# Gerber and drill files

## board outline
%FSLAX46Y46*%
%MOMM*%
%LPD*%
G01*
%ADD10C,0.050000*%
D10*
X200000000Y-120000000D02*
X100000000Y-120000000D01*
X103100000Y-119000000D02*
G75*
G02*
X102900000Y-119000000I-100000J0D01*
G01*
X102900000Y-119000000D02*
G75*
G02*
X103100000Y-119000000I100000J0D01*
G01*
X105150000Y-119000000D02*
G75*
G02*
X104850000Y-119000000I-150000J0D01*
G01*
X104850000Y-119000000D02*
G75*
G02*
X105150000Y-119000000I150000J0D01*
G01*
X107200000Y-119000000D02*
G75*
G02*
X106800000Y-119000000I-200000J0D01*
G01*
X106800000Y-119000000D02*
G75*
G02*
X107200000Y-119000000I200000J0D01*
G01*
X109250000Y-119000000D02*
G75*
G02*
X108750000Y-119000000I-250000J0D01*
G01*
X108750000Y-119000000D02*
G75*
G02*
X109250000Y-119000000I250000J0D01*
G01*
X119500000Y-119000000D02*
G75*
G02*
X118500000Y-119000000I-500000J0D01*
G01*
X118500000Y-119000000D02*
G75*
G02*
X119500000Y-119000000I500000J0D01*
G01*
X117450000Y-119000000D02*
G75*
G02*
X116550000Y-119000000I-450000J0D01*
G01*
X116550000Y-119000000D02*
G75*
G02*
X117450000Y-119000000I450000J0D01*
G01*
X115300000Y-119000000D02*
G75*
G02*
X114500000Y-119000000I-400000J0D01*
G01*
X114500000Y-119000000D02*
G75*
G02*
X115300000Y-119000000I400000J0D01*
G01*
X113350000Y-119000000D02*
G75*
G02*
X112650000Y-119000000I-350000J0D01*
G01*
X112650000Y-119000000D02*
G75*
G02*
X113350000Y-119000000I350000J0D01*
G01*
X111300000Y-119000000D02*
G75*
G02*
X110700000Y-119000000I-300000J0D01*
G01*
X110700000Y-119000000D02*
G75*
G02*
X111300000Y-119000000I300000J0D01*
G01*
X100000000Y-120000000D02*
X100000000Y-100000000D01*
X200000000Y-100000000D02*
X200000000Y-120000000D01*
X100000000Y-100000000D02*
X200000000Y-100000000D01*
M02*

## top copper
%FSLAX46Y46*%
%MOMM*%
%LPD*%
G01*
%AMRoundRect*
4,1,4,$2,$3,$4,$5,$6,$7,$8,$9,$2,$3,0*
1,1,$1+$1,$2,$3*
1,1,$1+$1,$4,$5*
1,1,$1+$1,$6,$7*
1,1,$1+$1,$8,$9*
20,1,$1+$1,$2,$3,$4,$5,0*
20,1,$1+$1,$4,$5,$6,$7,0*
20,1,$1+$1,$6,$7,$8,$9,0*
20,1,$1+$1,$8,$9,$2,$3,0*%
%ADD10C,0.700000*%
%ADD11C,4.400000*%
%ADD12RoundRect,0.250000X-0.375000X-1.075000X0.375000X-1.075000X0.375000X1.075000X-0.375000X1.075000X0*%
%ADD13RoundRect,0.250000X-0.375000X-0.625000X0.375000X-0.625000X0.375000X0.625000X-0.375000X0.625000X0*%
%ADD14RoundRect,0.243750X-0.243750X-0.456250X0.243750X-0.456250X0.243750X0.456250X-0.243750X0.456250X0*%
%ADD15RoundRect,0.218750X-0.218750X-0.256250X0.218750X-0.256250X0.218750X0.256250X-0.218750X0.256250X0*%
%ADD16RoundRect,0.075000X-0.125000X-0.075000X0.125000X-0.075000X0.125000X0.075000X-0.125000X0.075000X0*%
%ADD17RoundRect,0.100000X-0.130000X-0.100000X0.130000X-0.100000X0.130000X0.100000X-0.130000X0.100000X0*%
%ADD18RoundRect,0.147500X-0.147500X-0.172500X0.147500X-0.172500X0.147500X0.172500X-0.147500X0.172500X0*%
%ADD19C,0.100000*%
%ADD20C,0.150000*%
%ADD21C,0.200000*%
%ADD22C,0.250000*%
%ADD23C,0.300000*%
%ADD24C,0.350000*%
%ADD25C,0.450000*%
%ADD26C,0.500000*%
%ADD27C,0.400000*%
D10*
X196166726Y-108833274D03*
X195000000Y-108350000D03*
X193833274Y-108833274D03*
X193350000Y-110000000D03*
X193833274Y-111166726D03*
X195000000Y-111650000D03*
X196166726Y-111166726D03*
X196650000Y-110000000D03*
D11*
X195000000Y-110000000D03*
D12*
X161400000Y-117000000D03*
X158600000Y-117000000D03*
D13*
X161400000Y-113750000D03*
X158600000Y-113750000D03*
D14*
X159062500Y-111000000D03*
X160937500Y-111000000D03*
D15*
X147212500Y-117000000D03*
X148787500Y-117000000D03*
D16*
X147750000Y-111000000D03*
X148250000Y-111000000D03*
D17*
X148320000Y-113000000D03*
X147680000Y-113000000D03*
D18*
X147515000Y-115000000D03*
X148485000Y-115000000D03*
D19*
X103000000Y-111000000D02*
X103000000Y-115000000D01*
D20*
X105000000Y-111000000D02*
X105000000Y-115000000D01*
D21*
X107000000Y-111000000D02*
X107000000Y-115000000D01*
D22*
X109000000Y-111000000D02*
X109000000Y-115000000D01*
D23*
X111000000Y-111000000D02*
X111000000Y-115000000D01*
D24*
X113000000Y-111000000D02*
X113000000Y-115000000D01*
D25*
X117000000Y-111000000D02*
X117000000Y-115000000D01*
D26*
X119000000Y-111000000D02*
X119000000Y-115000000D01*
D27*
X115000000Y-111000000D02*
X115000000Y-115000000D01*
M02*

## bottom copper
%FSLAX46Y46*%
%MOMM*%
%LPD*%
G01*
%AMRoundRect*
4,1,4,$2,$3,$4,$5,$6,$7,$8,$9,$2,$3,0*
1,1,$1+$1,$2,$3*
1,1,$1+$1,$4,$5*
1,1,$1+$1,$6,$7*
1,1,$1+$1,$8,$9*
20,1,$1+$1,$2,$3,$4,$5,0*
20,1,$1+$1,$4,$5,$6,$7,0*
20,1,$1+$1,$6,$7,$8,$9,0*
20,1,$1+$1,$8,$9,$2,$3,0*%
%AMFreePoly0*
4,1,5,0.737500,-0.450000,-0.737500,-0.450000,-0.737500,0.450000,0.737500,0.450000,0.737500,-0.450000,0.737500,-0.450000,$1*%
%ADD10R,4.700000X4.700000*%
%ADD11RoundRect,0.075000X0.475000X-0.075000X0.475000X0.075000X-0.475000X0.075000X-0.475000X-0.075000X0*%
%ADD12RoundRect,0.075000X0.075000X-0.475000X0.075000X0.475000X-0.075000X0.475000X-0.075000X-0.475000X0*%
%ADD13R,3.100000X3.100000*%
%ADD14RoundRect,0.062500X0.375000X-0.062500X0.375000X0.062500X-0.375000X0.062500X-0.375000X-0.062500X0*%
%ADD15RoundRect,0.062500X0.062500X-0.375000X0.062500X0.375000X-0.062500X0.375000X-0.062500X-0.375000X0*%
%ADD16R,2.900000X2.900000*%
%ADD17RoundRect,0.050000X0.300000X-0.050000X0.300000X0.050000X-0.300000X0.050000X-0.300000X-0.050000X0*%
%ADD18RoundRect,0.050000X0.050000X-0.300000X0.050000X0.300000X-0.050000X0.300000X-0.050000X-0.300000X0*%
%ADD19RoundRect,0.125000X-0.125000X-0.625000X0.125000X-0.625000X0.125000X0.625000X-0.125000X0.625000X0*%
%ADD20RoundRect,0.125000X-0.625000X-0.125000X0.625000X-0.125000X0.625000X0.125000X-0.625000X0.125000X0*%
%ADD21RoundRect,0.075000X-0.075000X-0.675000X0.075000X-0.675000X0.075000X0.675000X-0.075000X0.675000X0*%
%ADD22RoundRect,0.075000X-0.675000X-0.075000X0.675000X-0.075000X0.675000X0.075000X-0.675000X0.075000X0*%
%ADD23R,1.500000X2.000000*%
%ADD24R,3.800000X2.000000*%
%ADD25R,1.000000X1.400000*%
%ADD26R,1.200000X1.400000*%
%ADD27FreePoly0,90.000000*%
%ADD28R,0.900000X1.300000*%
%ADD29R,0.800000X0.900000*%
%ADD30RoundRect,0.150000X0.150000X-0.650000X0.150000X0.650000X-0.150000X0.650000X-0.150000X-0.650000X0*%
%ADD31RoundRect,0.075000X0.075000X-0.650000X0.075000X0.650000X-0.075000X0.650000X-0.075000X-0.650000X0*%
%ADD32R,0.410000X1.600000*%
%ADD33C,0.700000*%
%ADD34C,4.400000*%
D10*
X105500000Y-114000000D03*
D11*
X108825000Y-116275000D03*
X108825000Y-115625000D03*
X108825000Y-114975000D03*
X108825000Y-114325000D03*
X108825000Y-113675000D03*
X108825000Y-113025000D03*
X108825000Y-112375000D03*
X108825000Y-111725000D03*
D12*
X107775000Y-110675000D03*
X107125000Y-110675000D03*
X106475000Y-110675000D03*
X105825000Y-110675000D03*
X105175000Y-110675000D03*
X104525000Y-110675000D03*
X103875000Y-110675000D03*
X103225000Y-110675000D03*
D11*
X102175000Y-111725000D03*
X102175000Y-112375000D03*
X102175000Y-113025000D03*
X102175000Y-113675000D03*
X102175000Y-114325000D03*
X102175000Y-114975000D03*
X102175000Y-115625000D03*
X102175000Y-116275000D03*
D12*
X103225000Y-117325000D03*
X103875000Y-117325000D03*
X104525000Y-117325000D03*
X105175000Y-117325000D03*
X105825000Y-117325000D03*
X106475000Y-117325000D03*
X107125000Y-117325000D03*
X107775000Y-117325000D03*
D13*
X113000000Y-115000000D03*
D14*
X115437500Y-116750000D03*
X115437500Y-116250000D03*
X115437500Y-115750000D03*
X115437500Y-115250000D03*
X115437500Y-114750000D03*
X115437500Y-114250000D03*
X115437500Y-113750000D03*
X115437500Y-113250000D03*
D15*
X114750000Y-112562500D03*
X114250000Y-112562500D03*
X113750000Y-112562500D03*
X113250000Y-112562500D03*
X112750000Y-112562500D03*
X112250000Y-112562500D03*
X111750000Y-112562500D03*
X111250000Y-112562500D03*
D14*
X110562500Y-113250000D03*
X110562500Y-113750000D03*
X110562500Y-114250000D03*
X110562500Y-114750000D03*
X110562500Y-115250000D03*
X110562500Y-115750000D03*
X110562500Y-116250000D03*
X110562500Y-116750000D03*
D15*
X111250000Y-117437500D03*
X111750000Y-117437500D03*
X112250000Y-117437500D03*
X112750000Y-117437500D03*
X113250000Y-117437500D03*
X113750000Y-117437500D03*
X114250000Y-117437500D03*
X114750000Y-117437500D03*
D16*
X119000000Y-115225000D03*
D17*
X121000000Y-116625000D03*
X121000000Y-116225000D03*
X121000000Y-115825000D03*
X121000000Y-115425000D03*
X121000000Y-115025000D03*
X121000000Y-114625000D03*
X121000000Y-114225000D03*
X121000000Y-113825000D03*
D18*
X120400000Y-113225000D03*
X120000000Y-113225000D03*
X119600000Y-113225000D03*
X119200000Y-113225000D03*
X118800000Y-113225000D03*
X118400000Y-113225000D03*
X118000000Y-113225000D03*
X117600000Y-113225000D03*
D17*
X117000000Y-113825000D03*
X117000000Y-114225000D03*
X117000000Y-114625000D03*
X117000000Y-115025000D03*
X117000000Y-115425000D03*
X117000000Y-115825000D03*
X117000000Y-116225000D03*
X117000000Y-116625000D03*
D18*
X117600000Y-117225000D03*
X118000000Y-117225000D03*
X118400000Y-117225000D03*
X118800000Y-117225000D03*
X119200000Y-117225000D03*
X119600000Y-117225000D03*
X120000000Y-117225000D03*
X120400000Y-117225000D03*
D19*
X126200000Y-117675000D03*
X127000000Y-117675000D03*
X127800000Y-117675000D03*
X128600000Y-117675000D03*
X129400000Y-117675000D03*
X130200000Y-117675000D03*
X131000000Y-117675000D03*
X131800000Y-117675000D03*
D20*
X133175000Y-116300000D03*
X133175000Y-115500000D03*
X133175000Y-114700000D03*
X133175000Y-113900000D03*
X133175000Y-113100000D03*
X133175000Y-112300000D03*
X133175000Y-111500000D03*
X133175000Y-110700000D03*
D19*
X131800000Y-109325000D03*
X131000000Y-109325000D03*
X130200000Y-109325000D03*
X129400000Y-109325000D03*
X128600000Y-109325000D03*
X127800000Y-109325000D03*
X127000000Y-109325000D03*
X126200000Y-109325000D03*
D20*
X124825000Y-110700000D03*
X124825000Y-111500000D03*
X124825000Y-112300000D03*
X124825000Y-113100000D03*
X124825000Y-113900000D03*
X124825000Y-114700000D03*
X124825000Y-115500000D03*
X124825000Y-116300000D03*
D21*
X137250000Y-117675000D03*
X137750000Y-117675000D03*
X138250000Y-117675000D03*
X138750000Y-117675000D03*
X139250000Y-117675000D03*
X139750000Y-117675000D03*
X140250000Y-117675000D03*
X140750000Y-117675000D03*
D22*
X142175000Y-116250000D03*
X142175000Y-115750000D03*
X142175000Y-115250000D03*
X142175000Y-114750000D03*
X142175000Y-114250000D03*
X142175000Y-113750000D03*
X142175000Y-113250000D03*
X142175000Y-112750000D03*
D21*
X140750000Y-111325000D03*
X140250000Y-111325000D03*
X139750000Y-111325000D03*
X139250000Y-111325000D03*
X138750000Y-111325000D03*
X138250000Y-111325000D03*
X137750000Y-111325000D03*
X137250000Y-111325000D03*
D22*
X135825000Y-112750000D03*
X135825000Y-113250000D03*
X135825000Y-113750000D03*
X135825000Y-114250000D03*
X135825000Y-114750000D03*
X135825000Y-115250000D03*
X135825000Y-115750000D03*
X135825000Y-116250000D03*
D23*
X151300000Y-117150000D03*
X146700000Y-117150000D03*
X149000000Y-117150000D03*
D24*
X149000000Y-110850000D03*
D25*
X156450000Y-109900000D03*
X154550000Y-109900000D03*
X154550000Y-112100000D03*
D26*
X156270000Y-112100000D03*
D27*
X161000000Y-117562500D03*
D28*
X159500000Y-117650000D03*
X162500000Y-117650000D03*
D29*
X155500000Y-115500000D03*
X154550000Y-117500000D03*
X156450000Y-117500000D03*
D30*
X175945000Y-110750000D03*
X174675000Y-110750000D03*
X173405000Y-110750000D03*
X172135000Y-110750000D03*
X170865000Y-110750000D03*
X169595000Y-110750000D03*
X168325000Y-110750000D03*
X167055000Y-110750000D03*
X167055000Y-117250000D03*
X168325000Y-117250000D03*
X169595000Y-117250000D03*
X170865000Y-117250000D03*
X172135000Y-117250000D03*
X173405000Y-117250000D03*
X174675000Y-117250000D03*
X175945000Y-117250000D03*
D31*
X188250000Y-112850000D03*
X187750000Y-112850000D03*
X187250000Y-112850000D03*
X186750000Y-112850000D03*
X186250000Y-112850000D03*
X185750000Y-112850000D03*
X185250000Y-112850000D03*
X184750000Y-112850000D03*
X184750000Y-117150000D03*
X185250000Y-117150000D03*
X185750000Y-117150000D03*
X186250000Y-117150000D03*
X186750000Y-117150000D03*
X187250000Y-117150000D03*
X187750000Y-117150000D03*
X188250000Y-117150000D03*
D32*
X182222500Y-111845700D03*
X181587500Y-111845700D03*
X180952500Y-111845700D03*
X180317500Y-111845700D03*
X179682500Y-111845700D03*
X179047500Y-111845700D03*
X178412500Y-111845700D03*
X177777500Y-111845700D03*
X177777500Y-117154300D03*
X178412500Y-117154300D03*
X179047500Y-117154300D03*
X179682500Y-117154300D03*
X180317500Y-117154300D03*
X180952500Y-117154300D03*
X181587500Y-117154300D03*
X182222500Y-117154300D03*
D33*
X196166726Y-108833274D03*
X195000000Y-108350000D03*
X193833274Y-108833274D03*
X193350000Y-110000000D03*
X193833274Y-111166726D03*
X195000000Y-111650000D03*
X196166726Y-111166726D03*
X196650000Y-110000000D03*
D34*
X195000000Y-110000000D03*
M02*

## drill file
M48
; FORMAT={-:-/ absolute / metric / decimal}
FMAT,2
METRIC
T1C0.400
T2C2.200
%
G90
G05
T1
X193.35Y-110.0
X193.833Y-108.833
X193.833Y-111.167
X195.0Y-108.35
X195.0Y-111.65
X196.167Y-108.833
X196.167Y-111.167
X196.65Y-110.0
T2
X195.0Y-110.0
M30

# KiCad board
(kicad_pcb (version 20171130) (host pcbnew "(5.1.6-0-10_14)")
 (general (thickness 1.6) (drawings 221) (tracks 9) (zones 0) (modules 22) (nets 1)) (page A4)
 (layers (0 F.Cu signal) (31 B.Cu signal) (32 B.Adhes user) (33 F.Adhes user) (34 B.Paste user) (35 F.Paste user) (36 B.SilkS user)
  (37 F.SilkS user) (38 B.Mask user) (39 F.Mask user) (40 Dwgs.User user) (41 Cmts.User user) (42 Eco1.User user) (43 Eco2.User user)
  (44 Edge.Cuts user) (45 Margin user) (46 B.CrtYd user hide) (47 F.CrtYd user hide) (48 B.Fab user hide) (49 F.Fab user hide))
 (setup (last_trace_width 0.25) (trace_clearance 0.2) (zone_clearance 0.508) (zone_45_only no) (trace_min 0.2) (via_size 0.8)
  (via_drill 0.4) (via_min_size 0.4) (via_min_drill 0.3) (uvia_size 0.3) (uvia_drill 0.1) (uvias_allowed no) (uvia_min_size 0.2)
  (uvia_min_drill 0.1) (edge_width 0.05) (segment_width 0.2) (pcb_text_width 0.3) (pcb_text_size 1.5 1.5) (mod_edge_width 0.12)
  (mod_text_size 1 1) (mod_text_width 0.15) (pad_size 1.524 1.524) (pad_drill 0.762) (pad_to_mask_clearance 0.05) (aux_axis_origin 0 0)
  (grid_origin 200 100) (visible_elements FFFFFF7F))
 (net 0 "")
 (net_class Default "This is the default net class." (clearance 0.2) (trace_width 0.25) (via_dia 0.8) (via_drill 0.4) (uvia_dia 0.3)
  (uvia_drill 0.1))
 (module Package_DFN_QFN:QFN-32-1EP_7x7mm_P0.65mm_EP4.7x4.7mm (layer B.Cu) (at 105.5 114 90)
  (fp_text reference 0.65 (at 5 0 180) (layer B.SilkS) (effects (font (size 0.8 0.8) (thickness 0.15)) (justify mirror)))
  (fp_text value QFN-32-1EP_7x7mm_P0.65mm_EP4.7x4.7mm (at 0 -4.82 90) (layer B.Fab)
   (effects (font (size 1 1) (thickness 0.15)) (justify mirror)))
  (pad "" smd roundrect (at 1.77 -1.77 90) (size 0.95 0.95) (layers B.Paste) (roundrect_rratio 0.25))
  (pad "" smd roundrect (at 1.77 -0.59 90) (size 0.95 0.95) (layers B.Paste) (roundrect_rratio 0.25))
  (pad "" smd roundrect (at 1.77 0.59 90) (size 0.95 0.95) (layers B.Paste) (roundrect_rratio 0.25))
  (pad "" smd roundrect (at 1.77 1.77 90) (size 0.95 0.95) (layers B.Paste) (roundrect_rratio 0.25))
  (pad "" smd roundrect (at 0.59 -1.77 90) (size 0.95 0.95) (layers B.Paste) (roundrect_rratio 0.25))
  (pad "" smd roundrect (at 0.59 -0.59 90) (size 0.95 0.95) (layers B.Paste) (roundrect_rratio 0.25))
  (pad "" smd roundrect (at 0.59 0.59 90) (size 0.95 0.95) (layers B.Paste) (roundrect_rratio 0.25))
  (pad "" smd roundrect (at 0.59 1.77 90) (size 0.95 0.95) (layers B.Paste) (roundrect_rratio 0.25))
  (pad "" smd roundrect (at -0.59 -1.77 90) (size 0.95 0.95) (layers B.Paste) (roundrect_rratio 0.25))
  (pad "" smd roundrect (at -0.59 -0.59 90) (size 0.95 0.95) (layers B.Paste) (roundrect_rratio 0.25))
  (pad "" smd roundrect (at -0.59 0.59 90) (size 0.95 0.95) (layers B.Paste) (roundrect_rratio 0.25))
  (pad "" smd roundrect (at -0.59 1.77 90) (size 0.95 0.95) (layers B.Paste) (roundrect_rratio 0.25))
  (pad "" smd roundrect (at -1.77 -1.77 90) (size 0.95 0.95) (layers B.Paste) (roundrect_rratio 0.25))
  (pad "" smd roundrect (at -1.77 -0.59 90) (size 0.95 0.95) (layers B.Paste) (roundrect_rratio 0.25))
  (pad "" smd roundrect (at -1.77 0.59 90) (size 0.95 0.95) (layers B.Paste) (roundrect_rratio 0.25))
  (pad "" smd roundrect (at -1.77 1.77 90) (size 0.95 0.95) (layers B.Paste) (roundrect_rratio 0.25))
  (pad 33 smd rect (at 0 0 90) (size 4.7 4.7) (layers B.Cu B.Mask))
  (pad 32 smd roundrect (at -2.275 3.325 90) (size 0.3 1.1) (layers B.Cu B.Paste B.Mask) (roundrect_rratio 0.25))
  (pad 31 smd roundrect (at -1.625 3.325 90) (size 0.3 1.1) (layers B.Cu B.Paste B.Mask) (roundrect_rratio 0.25))
  (pad 30 smd roundrect (at -0.975 3.325 90) (size 0.3 1.1) (layers B.Cu B.Paste B.Mask) (roundrect_rratio 0.25))
  (pad 29 smd roundrect (at -0.325 3.325 90) (size 0.3 1.1) (layers B.Cu B.Paste B.Mask) (roundrect_rratio 0.25))
  (pad 28 smd roundrect (at 0.325 3.325 90) (size 0.3 1.1) (layers B.Cu B.Paste B.Mask) (roundrect_rratio 0.25))
  (pad 27 smd roundrect (at 0.975 3.325 90) (size 0.3 1.1) (layers B.Cu B.Paste B.Mask) (roundrect_rratio 0.25))
  (pad 26 smd roundrect (at 1.625 3.325 90) (size 0.3 1.1) (layers B.Cu B.Paste B.Mask) (roundrect_rratio 0.25))
  (pad 25 smd roundrect (at 2.275 3.325 90) (size 0.3 1.1) (layers B.Cu B.Paste B.Mask) (roundrect_rratio 0.25))
  (pad 24 smd roundrect (at 3.325 2.275 90) (size 1.1 0.3) (layers B.Cu B.Paste B.Mask) (roundrect_rratio 0.25))
  (pad 23 smd roundrect (at 3.325 1.625 90) (size 1.1 0.3) (layers B.Cu B.Paste B.Mask) (roundrect_rratio 0.25))
  (pad 22 smd roundrect (at 3.325 0.975 90) (size 1.1 0.3) (layers B.Cu B.Paste B.Mask) (roundrect_rratio 0.25))
  (pad 21 smd roundrect (at 3.325 0.325 90) (size 1.1 0.3) (layers B.Cu B.Paste B.Mask) (roundrect_rratio 0.25))
  (pad 20 smd roundrect (at 3.325 -0.325 90) (size 1.1 0.3) (layers B.Cu B.Paste B.Mask) (roundrect_rratio 0.25))
  (pad 19 smd roundrect (at 3.325 -0.975 90) (size 1.1 0.3) (layers B.Cu B.Paste B.Mask) (roundrect_rratio 0.25))
  (pad 18 smd roundrect (at 3.325 -1.625 90) (size 1.1 0.3) (layers B.Cu B.Paste B.Mask) (roundrect_rratio 0.25))
  (pad 17 smd roundrect (at 3.325 -2.275 90) (size 1.1 0.3) (layers B.Cu B.Paste B.Mask) (roundrect_rratio 0.25))
  (pad 16 smd roundrect (at 2.275 -3.325 90) (size 0.3 1.1) (layers B.Cu B.Paste B.Mask) (roundrect_rratio 0.25))
  (pad 15 smd roundrect (at 1.625 -3.325 90) (size 0.3 1.1) (layers B.Cu B.Paste B.Mask) (roundrect_rratio 0.25))
  (pad 14 smd roundrect (at 0.975 -3.325 90) (size 0.3 1.1) (layers B.Cu B.Paste B.Mask) (roundrect_rratio 0.25))
  (pad 13 smd roundrect (at 0.325 -3.325 90) (size 0.3 1.1) (layers B.Cu B.Paste B.Mask) (roundrect_rratio 0.25))
  (pad 12 smd roundrect (at -0.325 -3.325 90) (size 0.3 1.1) (layers B.Cu B.Paste B.Mask) (roundrect_rratio 0.25))
  (pad 11 smd roundrect (at -0.975 -3.325 90) (size 0.3 1.1) (layers B.Cu B.Paste B.Mask) (roundrect_rratio 0.25))
  (pad 10 smd roundrect (at -1.625 -3.325 90) (size 0.3 1.1) (layers B.Cu B.Paste B.Mask) (roundrect_rratio 0.25))
  (pad 9 smd roundrect (at -2.275 -3.325 90) (size 0.3 1.1) (layers B.Cu B.Paste B.Mask) (roundrect_rratio 0.25))
  (pad 8 smd roundrect (at -3.325 -2.275 90) (size 1.1 0.3) (layers B.Cu B.Paste B.Mask) (roundrect_rratio 0.25))
  (pad 7 smd roundrect (at -3.325 -1.625 90) (size 1.1 0.3) (layers B.Cu B.Paste B.Mask) (roundrect_rratio 0.25))
  (pad 6 smd roundrect (at -3.325 -0.975 90) (size 1.1 0.3) (layers B.Cu B.Paste B.Mask) (roundrect_rratio 0.25))
  (pad 5 smd roundrect (at -3.325 -0.325 90) (size 1.1 0.3) (layers B.Cu B.Paste B.Mask) (roundrect_rratio 0.25))
  (pad 4 smd roundrect (at -3.325 0.325 90) (size 1.1 0.3) (layers B.Cu B.Paste B.Mask) (roundrect_rratio 0.25))
  (pad 3 smd roundrect (at -3.325 0.975 90) (size 1.1 0.3) (layers B.Cu B.Paste B.Mask) (roundrect_rratio 0.25))
  (pad 2 smd roundrect (at -3.325 1.625 90) (size 1.1 0.3) (layers B.Cu B.Paste B.Mask) (roundrect_rratio 0.25))
  (pad 1 smd roundrect (at -3.325 2.275 90) (size 1.1 0.3) (layers B.Cu B.Paste B.Mask) (roundrect_rratio 0.25)))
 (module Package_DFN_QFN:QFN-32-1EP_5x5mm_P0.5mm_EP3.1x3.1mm (layer B.Cu) (at 113 115 90)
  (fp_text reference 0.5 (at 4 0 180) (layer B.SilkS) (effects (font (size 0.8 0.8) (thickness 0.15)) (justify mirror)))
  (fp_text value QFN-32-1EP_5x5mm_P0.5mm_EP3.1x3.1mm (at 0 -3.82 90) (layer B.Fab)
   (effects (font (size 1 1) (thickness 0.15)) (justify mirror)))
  (pad "" smd roundrect (at 1.03 -1.03 90) (size 0.83 0.83) (layers B.Paste) (roundrect_rratio 0.25))
  (pad "" smd roundrect (at 1.03 0 90) (size 0.83 0.83) (layers B.Paste) (roundrect_rratio 0.25))
  (pad "" smd roundrect (at 1.03 1.03 90) (size 0.83 0.83) (layers B.Paste) (roundrect_rratio 0.25))
  (pad "" smd roundrect (at 0 -1.03 90) (size 0.83 0.83) (layers B.Paste) (roundrect_rratio 0.25))
  (pad "" smd roundrect (at 0 0 90) (size 0.83 0.83) (layers B.Paste) (roundrect_rratio 0.25))
  (pad "" smd roundrect (at 0 1.03 90) (size 0.83 0.83) (layers B.Paste) (roundrect_rratio 0.25))
  (pad "" smd roundrect (at -1.03 -1.03 90) (size 0.83 0.83) (layers B.Paste) (roundrect_rratio 0.25))
  (pad "" smd roundrect (at -1.03 0 90) (size 0.83 0.83) (layers B.Paste) (roundrect_rratio 0.25))
  (pad "" smd roundrect (at -1.03 1.03 90) (size 0.83 0.83) (layers B.Paste) (roundrect_rratio 0.25))
  (pad 33 smd rect (at 0 0 90) (size 3.1 3.1) (layers B.Cu B.Mask))
  (pad 32 smd roundrect (at -1.75 2.4375 90) (size 0.25 0.875) (layers B.Cu B.Paste B.Mask) (roundrect_rratio 0.25))
  (pad 31 smd roundrect (at -1.25 2.4375 90) (size 0.25 0.875) (layers B.Cu B.Paste B.Mask) (roundrect_rratio 0.25))
  (pad 30 smd roundrect (at -0.75 2.4375 90) (size 0.25 0.875) (layers B.Cu B.Paste B.Mask) (roundrect_rratio 0.25))
  (pad 29 smd roundrect (at -0.25 2.4375 90) (size 0.25 0.875) (layers B.Cu B.Paste B.Mask) (roundrect_rratio 0.25))
  (pad 28 smd roundrect (at 0.25 2.4375 90) (size 0.25 0.875) (layers B.Cu B.Paste B.Mask) (roundrect_rratio 0.25))
  (pad 27 smd roundrect (at 0.75 2.4375 90) (size 0.25 0.875) (layers B.Cu B.Paste B.Mask) (roundrect_rratio 0.25))
  (pad 26 smd roundrect (at 1.25 2.4375 90) (size 0.25 0.875) (layers B.Cu B.Paste B.Mask) (roundrect_rratio 0.25))
  (pad 25 smd roundrect (at 1.75 2.4375 90) (size 0.25 0.875) (layers B.Cu B.Paste B.Mask) (roundrect_rratio 0.25))
  (pad 24 smd roundrect (at 2.4375 1.75 90) (size 0.875 0.25) (layers B.Cu B.Paste B.Mask) (roundrect_rratio 0.25))
  (pad 23 smd roundrect (at 2.4375 1.25 90) (size 0.875 0.25) (layers B.Cu B.Paste B.Mask) (roundrect_rratio 0.25))
  (pad 22 smd roundrect (at 2.4375 0.75 90) (size 0.875 0.25) (layers B.Cu B.Paste B.Mask) (roundrect_rratio 0.25))
  (pad 21 smd roundrect (at 2.4375 0.25 90) (size 0.875 0.25) (layers B.Cu B.Paste B.Mask) (roundrect_rratio 0.25))
  (pad 20 smd roundrect (at 2.4375 -0.25 90) (size 0.875 0.25) (layers B.Cu B.Paste B.Mask) (roundrect_rratio 0.25))
  (pad 19 smd roundrect (at 2.4375 -0.75 90) (size 0.875 0.25) (layers B.Cu B.Paste B.Mask) (roundrect_rratio 0.25))
  (pad 18 smd roundrect (at 2.4375 -1.25 90) (size 0.875 0.25) (layers B.Cu B.Paste B.Mask) (roundrect_rratio 0.25))
  (pad 17 smd roundrect (at 2.4375 -1.75 90) (size 0.875 0.25) (layers B.Cu B.Paste B.Mask) (roundrect_rratio 0.25))
  (pad 16 smd roundrect (at 1.75 -2.4375 90) (size 0.25 0.875) (layers B.Cu B.Paste B.Mask) (roundrect_rratio 0.25))
  (pad 15 smd roundrect (at 1.25 -2.4375 90) (size 0.25 0.875) (layers B.Cu B.Paste B.Mask) (roundrect_rratio 0.25))
  (pad 14 smd roundrect (at 0.75 -2.4375 90) (size 0.25 0.875) (layers B.Cu B.Paste B.Mask) (roundrect_rratio 0.25))
  (pad 13 smd roundrect (at 0.25 -2.4375 90) (size 0.25 0.875) (layers B.Cu B.Paste B.Mask) (roundrect_rratio 0.25))
  (pad 12 smd roundrect (at -0.25 -2.4375 90) (size 0.25 0.875) (layers B.Cu B.Paste B.Mask) (roundrect_rratio 0.25))
  (pad 11 smd roundrect (at -0.75 -2.4375 90) (size 0.25 0.875) (layers B.Cu B.Paste B.Mask) (roundrect_rratio 0.25))
  (pad 10 smd roundrect (at -1.25 -2.4375 90) (size 0.25 0.875) (layers B.Cu B.Paste B.Mask) (roundrect_rratio 0.25))
  (pad 9 smd roundrect (at -1.75 -2.4375 90) (size 0.25 0.875) (layers B.Cu B.Paste B.Mask) (roundrect_rratio 0.25))
  (pad 8 smd roundrect (at -2.4375 -1.75 90) (size 0.875 0.25) (layers B.Cu B.Paste B.Mask) (roundrect_rratio 0.25))
  (pad 7 smd roundrect (at -2.4375 -1.25 90) (size 0.875 0.25) (layers B.Cu B.Paste B.Mask) (roundrect_rratio 0.25))
  (pad 6 smd roundrect (at -2.4375 -0.75 90) (size 0.875 0.25) (layers B.Cu B.Paste B.Mask) (roundrect_rratio 0.25))
  (pad 5 smd roundrect (at -2.4375 -0.25 90) (size 0.875 0.25) (layers B.Cu B.Paste B.Mask) (roundrect_rratio 0.25))
  (pad 4 smd roundrect (at -2.4375 0.25 90) (size 0.875 0.25) (layers B.Cu B.Paste B.Mask) (roundrect_rratio 0.25))
  (pad 3 smd roundrect (at -2.4375 0.75 90) (size 0.875 0.25) (layers B.Cu B.Paste B.Mask) (roundrect_rratio 0.25))
  (pad 2 smd roundrect (at -2.4375 1.25 90) (size 0.875 0.25) (layers B.Cu B.Paste B.Mask) (roundrect_rratio 0.25))
  (pad 1 smd roundrect (at -2.4375 1.75 90) (size 0.875 0.25) (layers B.Cu B.Paste B.Mask) (roundrect_rratio 0.25)))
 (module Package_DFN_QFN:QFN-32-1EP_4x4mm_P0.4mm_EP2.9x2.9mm (layer B.Cu) (at 119 115.225 90)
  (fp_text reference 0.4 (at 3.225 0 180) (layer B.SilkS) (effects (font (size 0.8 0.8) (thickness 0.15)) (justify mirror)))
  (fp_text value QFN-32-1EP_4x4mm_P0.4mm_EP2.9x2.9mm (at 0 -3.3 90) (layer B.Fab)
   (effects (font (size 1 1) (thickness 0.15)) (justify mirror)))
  (pad "" smd roundrect (at 0.725 -0.725 90) (size 1.17 1.17) (layers B.Paste) (roundrect_rratio 0.213675))
  (pad "" smd roundrect (at 0.725 0.725 90) (size 1.17 1.17) (layers B.Paste) (roundrect_rratio 0.213675))
  (pad "" smd roundrect (at -0.725 -0.725 90) (size 1.17 1.17) (layers B.Paste) (roundrect_rratio 0.213675))
  (pad "" smd roundrect (at -0.725 0.725 90) (size 1.17 1.17) (layers B.Paste) (roundrect_rratio 0.213675))
  (pad 33 smd rect (at 0 0 90) (size 2.9 2.9) (layers B.Cu B.Mask))
  (pad 32 smd roundrect (at -1.4 2 90) (size 0.2 0.7) (layers B.Cu B.Paste B.Mask) (roundrect_rratio 0.25))
  (pad 31 smd roundrect (at -1 2 90) (size 0.2 0.7) (layers B.Cu B.Paste B.Mask) (roundrect_rratio 0.25))
  (pad 30 smd roundrect (at -0.6 2 90) (size 0.2 0.7) (layers B.Cu B.Paste B.Mask) (roundrect_rratio 0.25))
  (pad 29 smd roundrect (at -0.2 2 90) (size 0.2 0.7) (layers B.Cu B.Paste B.Mask) (roundrect_rratio 0.25))
  (pad 28 smd roundrect (at 0.2 2 90) (size 0.2 0.7) (layers B.Cu B.Paste B.Mask) (roundrect_rratio 0.25))
  (pad 27 smd roundrect (at 0.6 2 90) (size 0.2 0.7) (layers B.Cu B.Paste B.Mask) (roundrect_rratio 0.25))
  (pad 26 smd roundrect (at 1 2 90) (size 0.2 0.7) (layers B.Cu B.Paste B.Mask) (roundrect_rratio 0.25))
  (pad 25 smd roundrect (at 1.4 2 90) (size 0.2 0.7) (layers B.Cu B.Paste B.Mask) (roundrect_rratio 0.25))
  (pad 24 smd roundrect (at 2 1.4 90) (size 0.7 0.2) (layers B.Cu B.Paste B.Mask) (roundrect_rratio 0.25))
  (pad 23 smd roundrect (at 2 1 90) (size 0.7 0.2) (layers B.Cu B.Paste B.Mask) (roundrect_rratio 0.25))
  (pad 22 smd roundrect (at 2 0.6 90) (size 0.7 0.2) (layers B.Cu B.Paste B.Mask) (roundrect_rratio 0.25))
  (pad 21 smd roundrect (at 2 0.2 90) (size 0.7 0.2) (layers B.Cu B.Paste B.Mask) (roundrect_rratio 0.25))
  (pad 20 smd roundrect (at 2 -0.2 90) (size 0.7 0.2) (layers B.Cu B.Paste B.Mask) (roundrect_rratio 0.25))
  (pad 19 smd roundrect (at 2 -0.6 90) (size 0.7 0.2) (layers B.Cu B.Paste B.Mask) (roundrect_rratio 0.25))
  (pad 18 smd roundrect (at 2 -1 90) (size 0.7 0.2) (layers B.Cu B.Paste B.Mask) (roundrect_rratio 0.25))
  (pad 17 smd roundrect (at 2 -1.4 90) (size 0.7 0.2) (layers B.Cu B.Paste B.Mask) (roundrect_rratio 0.25))
  (pad 16 smd roundrect (at 1.4 -2 90) (size 0.2 0.7) (layers B.Cu B.Paste B.Mask) (roundrect_rratio 0.25))
  (pad 15 smd roundrect (at 1 -2 90) (size 0.2 0.7) (layers B.Cu B.Paste B.Mask) (roundrect_rratio 0.25))
  (pad 14 smd roundrect (at 0.6 -2 90) (size 0.2 0.7) (layers B.Cu B.Paste B.Mask) (roundrect_rratio 0.25))
  (pad 13 smd roundrect (at 0.2 -2 90) (size 0.2 0.7) (layers B.Cu B.Paste B.Mask) (roundrect_rratio 0.25))
  (pad 12 smd roundrect (at -0.2 -2 90) (size 0.2 0.7) (layers B.Cu B.Paste B.Mask) (roundrect_rratio 0.25))
  (pad 11 smd roundrect (at -0.6 -2 90) (size 0.2 0.7) (layers B.Cu B.Paste B.Mask) (roundrect_rratio 0.25))
  (pad 10 smd roundrect (at -1 -2 90) (size 0.2 0.7) (layers B.Cu B.Paste B.Mask) (roundrect_rratio 0.25))
  (pad 9 smd roundrect (at -1.4 -2 90) (size 0.2 0.7) (layers B.Cu B.Paste B.Mask) (roundrect_rratio 0.25))
  (pad 8 smd roundrect (at -2 -1.4 90) (size 0.7 0.2) (layers B.Cu B.Paste B.Mask) (roundrect_rratio 0.25))
  (pad 7 smd roundrect (at -2 -1 90) (size 0.7 0.2) (layers B.Cu B.Paste B.Mask) (roundrect_rratio 0.25))
  (pad 6 smd roundrect (at -2 -0.6 90) (size 0.7 0.2) (layers B.Cu B.Paste B.Mask) (roundrect_rratio 0.25))
  (pad 5 smd roundrect (at -2 -0.2 90) (size 0.7 0.2) (layers B.Cu B.Paste B.Mask) (roundrect_rratio 0.25))
  (pad 4 smd roundrect (at -2 0.2 90) (size 0.7 0.2) (layers B.Cu B.Paste B.Mask) (roundrect_rratio 0.25))
  (pad 3 smd roundrect (at -2 0.6 90) (size 0.7 0.2) (layers B.Cu B.Paste B.Mask) (roundrect_rratio 0.25))
  (pad 2 smd roundrect (at -2 1 90) (size 0.7 0.2) (layers B.Cu B.Paste B.Mask) (roundrect_rratio 0.25))
  (pad 1 smd roundrect (at -2 1.4 90) (size 0.7 0.2) (layers B.Cu B.Paste B.Mask) (roundrect_rratio 0.25)))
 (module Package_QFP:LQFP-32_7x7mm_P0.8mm (layer B.Cu) (at 129 113.5)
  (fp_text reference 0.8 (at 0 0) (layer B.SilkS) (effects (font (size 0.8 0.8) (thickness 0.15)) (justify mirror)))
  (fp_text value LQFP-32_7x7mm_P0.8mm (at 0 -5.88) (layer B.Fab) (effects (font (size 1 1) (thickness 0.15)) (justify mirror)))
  (pad 32 smd roundrect (at -2.8 4.175) (size 0.5 1.5) (layers B.Cu B.Paste B.Mask) (roundrect_rratio 0.25))
  (pad 31 smd roundrect (at -2 4.175) (size 0.5 1.5) (layers B.Cu B.Paste B.Mask) (roundrect_rratio 0.25))
  (pad 30 smd roundrect (at -1.2 4.175) (size 0.5 1.5) (layers B.Cu B.Paste B.Mask) (roundrect_rratio 0.25))
  (pad 29 smd roundrect (at -0.4 4.175) (size 0.5 1.5) (layers B.Cu B.Paste B.Mask) (roundrect_rratio 0.25))
  (pad 28 smd roundrect (at 0.4 4.175) (size 0.5 1.5) (layers B.Cu B.Paste B.Mask) (roundrect_rratio 0.25))
  (pad 27 smd roundrect (at 1.2 4.175) (size 0.5 1.5) (layers B.Cu B.Paste B.Mask) (roundrect_rratio 0.25))
  (pad 26 smd roundrect (at 2 4.175) (size 0.5 1.5) (layers B.Cu B.Paste B.Mask) (roundrect_rratio 0.25))
  (pad 25 smd roundrect (at 2.8 4.175) (size 0.5 1.5) (layers B.Cu B.Paste B.Mask) (roundrect_rratio 0.25))
  (pad 24 smd roundrect (at 4.175 2.8) (size 1.5 0.5) (layers B.Cu B.Paste B.Mask) (roundrect_rratio 0.25))
  (pad 23 smd roundrect (at 4.175 2) (size 1.5 0.5) (layers B.Cu B.Paste B.Mask) (roundrect_rratio 0.25))
  (pad 22 smd roundrect (at 4.175 1.2) (size 1.5 0.5) (layers B.Cu B.Paste B.Mask) (roundrect_rratio 0.25))
  (pad 21 smd roundrect (at 4.175 0.4) (size 1.5 0.5) (layers B.Cu B.Paste B.Mask) (roundrect_rratio 0.25))
  (pad 20 smd roundrect (at 4.175 -0.4) (size 1.5 0.5) (layers B.Cu B.Paste B.Mask) (roundrect_rratio 0.25))
  (pad 19 smd roundrect (at 4.175 -1.2) (size 1.5 0.5) (layers B.Cu B.Paste B.Mask) (roundrect_rratio 0.25))
  (pad 18 smd roundrect (at 4.175 -2) (size 1.5 0.5) (layers B.Cu B.Paste B.Mask) (roundrect_rratio 0.25))
  (pad 17 smd roundrect (at 4.175 -2.8) (size 1.5 0.5) (layers B.Cu B.Paste B.Mask) (roundrect_rratio 0.25))
  (pad 16 smd roundrect (at 2.8 -4.175) (size 0.5 1.5) (layers B.Cu B.Paste B.Mask) (roundrect_rratio 0.25))
  (pad 15 smd roundrect (at 2 -4.175) (size 0.5 1.5) (layers B.Cu B.Paste B.Mask) (roundrect_rratio 0.25))
  (pad 14 smd roundrect (at 1.2 -4.175) (size 0.5 1.5) (layers B.Cu B.Paste B.Mask) (roundrect_rratio 0.25))
  (pad 13 smd roundrect (at 0.4 -4.175) (size 0.5 1.5) (layers B.Cu B.Paste B.Mask) (roundrect_rratio 0.25))
  (pad 12 smd roundrect (at -0.4 -4.175) (size 0.5 1.5) (layers B.Cu B.Paste B.Mask) (roundrect_rratio 0.25))
  (pad 11 smd roundrect (at -1.2 -4.175) (size 0.5 1.5) (layers B.Cu B.Paste B.Mask) (roundrect_rratio 0.25))
  (pad 10 smd roundrect (at -2 -4.175) (size 0.5 1.5) (layers B.Cu B.Paste B.Mask) (roundrect_rratio 0.25))
  (pad 9 smd roundrect (at -2.8 -4.175) (size 0.5 1.5) (layers B.Cu B.Paste B.Mask) (roundrect_rratio 0.25))
  (pad 8 smd roundrect (at -4.175 -2.8) (size 1.5 0.5) (layers B.Cu B.Paste B.Mask) (roundrect_rratio 0.25))
  (pad 7 smd roundrect (at -4.175 -2) (size 1.5 0.5) (layers B.Cu B.Paste B.Mask) (roundrect_rratio 0.25))
  (pad 6 smd roundrect (at -4.175 -1.2) (size 1.5 0.5) (layers B.Cu B.Paste B.Mask) (roundrect_rratio 0.25))
  (pad 5 smd roundrect (at -4.175 -0.4) (size 1.5 0.5) (layers B.Cu B.Paste B.Mask) (roundrect_rratio 0.25))
  (pad 4 smd roundrect (at -4.175 0.4) (size 1.5 0.5) (layers B.Cu B.Paste B.Mask) (roundrect_rratio 0.25))
  (pad 3 smd roundrect (at -4.175 1.2) (size 1.5 0.5) (layers B.Cu B.Paste B.Mask) (roundrect_rratio 0.25))
  (pad 2 smd roundrect (at -4.175 2) (size 1.5 0.5) (layers B.Cu B.Paste B.Mask) (roundrect_rratio 0.25))
  (pad 1 smd roundrect (at -4.175 2.8) (size 1.5 0.5) (layers B.Cu B.Paste B.Mask) (roundrect_rratio 0.25)))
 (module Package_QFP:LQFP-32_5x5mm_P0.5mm (layer B.Cu) (at 139 114.5)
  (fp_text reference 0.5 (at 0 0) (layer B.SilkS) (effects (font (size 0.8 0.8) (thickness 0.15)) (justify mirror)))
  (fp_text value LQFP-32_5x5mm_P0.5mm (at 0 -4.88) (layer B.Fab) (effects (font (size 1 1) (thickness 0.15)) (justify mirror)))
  (pad 32 smd roundrect (at -1.75 3.175) (size 0.3 1.5) (layers B.Cu B.Paste B.Mask) (roundrect_rratio 0.25))
  (pad 31 smd roundrect (at -1.25 3.175) (size 0.3 1.5) (layers B.Cu B.Paste B.Mask) (roundrect_rratio 0.25))
  (pad 30 smd roundrect (at -0.75 3.175) (size 0.3 1.5) (layers B.Cu B.Paste B.Mask) (roundrect_rratio 0.25))
  (pad 29 smd roundrect (at -0.25 3.175) (size 0.3 1.5) (layers B.Cu B.Paste B.Mask) (roundrect_rratio 0.25))
  (pad 28 smd roundrect (at 0.25 3.175) (size 0.3 1.5) (layers B.Cu B.Paste B.Mask) (roundrect_rratio 0.25))
  (pad 27 smd roundrect (at 0.75 3.175) (size 0.3 1.5) (layers B.Cu B.Paste B.Mask) (roundrect_rratio 0.25))
  (pad 26 smd roundrect (at 1.25 3.175) (size 0.3 1.5) (layers B.Cu B.Paste B.Mask) (roundrect_rratio 0.25))
  (pad 25 smd roundrect (at 1.75 3.175) (size 0.3 1.5) (layers B.Cu B.Paste B.Mask) (roundrect_rratio 0.25))
  (pad 24 smd roundrect (at 3.175 1.75) (size 1.5 0.3) (layers B.Cu B.Paste B.Mask) (roundrect_rratio 0.25))
  (pad 23 smd roundrect (at 3.175 1.25) (size 1.5 0.3) (layers B.Cu B.Paste B.Mask) (roundrect_rratio 0.25))
  (pad 22 smd roundrect (at 3.175 0.75) (size 1.5 0.3) (layers B.Cu B.Paste B.Mask) (roundrect_rratio 0.25))
  (pad 21 smd roundrect (at 3.175 0.25) (size 1.5 0.3) (layers B.Cu B.Paste B.Mask) (roundrect_rratio 0.25))
  (pad 20 smd roundrect (at 3.175 -0.25) (size 1.5 0.3) (layers B.Cu B.Paste B.Mask) (roundrect_rratio 0.25))
  (pad 19 smd roundrect (at 3.175 -0.75) (size 1.5 0.3) (layers B.Cu B.Paste B.Mask) (roundrect_rratio 0.25))
  (pad 18 smd roundrect (at 3.175 -1.25) (size 1.5 0.3) (layers B.Cu B.Paste B.Mask) (roundrect_rratio 0.25))
  (pad 17 smd roundrect (at 3.175 -1.75) (size 1.5 0.3) (layers B.Cu B.Paste B.Mask) (roundrect_rratio 0.25))
  (pad 16 smd roundrect (at 1.75 -3.175) (size 0.3 1.5) (layers B.Cu B.Paste B.Mask) (roundrect_rratio 0.25))
  (pad 15 smd roundrect (at 1.25 -3.175) (size 0.3 1.5) (layers B.Cu B.Paste B.Mask) (roundrect_rratio 0.25))
  (pad 14 smd roundrect (at 0.75 -3.175) (size 0.3 1.5) (layers B.Cu B.Paste B.Mask) (roundrect_rratio 0.25))
  (pad 13 smd roundrect (at 0.25 -3.175) (size 0.3 1.5) (layers B.Cu B.Paste B.Mask) (roundrect_rratio 0.25))
  (pad 12 smd roundrect (at -0.25 -3.175) (size 0.3 1.5) (layers B.Cu B.Paste B.Mask) (roundrect_rratio 0.25))
  (pad 11 smd roundrect (at -0.75 -3.175) (size 0.3 1.5) (layers B.Cu B.Paste B.Mask) (roundrect_rratio 0.25))
  (pad 10 smd roundrect (at -1.25 -3.175) (size 0.3 1.5) (layers B.Cu B.Paste B.Mask) (roundrect_rratio 0.25))
  (pad 9 smd roundrect (at -1.75 -3.175) (size 0.3 1.5) (layers B.Cu B.Paste B.Mask) (roundrect_rratio 0.25))
  (pad 8 smd roundrect (at -3.175 -1.75) (size 1.5 0.3) (layers B.Cu B.Paste B.Mask) (roundrect_rratio 0.25))
  (pad 7 smd roundrect (at -3.175 -1.25) (size 1.5 0.3) (layers B.Cu B.Paste B.Mask) (roundrect_rratio 0.25))
  (pad 6 smd roundrect (at -3.175 -0.75) (size 1.5 0.3) (layers B.Cu B.Paste B.Mask) (roundrect_rratio 0.25))
  (pad 5 smd roundrect (at -3.175 -0.25) (size 1.5 0.3) (layers B.Cu B.Paste B.Mask) (roundrect_rratio 0.25))
  (pad 4 smd roundrect (at -3.175 0.25) (size 1.5 0.3) (layers B.Cu B.Paste B.Mask) (roundrect_rratio 0.25))
  (pad 3 smd roundrect (at -3.175 0.75) (size 1.5 0.3) (layers B.Cu B.Paste B.Mask) (roundrect_rratio 0.25))
  (pad 2 smd roundrect (at -3.175 1.25) (size 1.5 0.3) (layers B.Cu B.Paste B.Mask) (roundrect_rratio 0.25))
  (pad 1 smd roundrect (at -3.175 1.75) (size 1.5 0.3) (layers B.Cu B.Paste B.Mask) (roundrect_rratio 0.25)))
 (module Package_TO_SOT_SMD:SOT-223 (layer B.Cu) (at 149 114 90)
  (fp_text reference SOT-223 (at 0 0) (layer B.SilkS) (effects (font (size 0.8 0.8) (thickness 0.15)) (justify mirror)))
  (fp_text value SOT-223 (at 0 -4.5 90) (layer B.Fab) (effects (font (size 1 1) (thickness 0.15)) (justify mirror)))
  (pad 1 smd rect (at -3.15 2.3 90) (size 2 1.5) (layers B.Cu B.Paste B.Mask))
  (pad 3 smd rect (at -3.15 -2.3 90) (size 2 1.5) (layers B.Cu B.Paste B.Mask))
  (pad 2 smd rect (at -3.15 0 90) (size 2 1.5) (layers B.Cu B.Paste B.Mask))
  (pad 4 smd rect (at 3.15 0 90) (size 2 3.8) (layers B.Cu B.Paste B.Mask)))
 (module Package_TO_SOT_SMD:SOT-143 (layer B.Cu) (at 155.5 111 90)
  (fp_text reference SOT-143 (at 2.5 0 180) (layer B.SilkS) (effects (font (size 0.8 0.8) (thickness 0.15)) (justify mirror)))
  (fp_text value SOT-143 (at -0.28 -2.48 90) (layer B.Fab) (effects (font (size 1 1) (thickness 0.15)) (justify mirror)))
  (pad 4 smd rect (at 1.1 0.95 180) (size 1 1.4) (layers B.Cu B.Paste B.Mask))
  (pad 3 smd rect (at 1.1 -0.95 180) (size 1 1.4) (layers B.Cu B.Paste B.Mask))
  (pad 2 smd rect (at -1.1 -0.95 180) (size 1 1.4) (layers B.Cu B.Paste B.Mask))
  (pad 1 smd rect (at -1.1 0.77 180) (size 1.2 1.4) (layers B.Cu B.Paste B.Mask)))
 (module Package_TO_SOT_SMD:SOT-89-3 (layer B.Cu) (at 161 116 90)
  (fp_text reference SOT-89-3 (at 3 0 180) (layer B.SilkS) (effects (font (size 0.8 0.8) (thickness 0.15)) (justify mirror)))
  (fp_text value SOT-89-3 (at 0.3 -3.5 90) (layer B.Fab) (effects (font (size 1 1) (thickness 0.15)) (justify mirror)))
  (pad 2 smd custom (at -1.5625 0 90) (size 1.475 0.9) (layers B.Cu B.Paste B.Mask) (zone_connect 2)
   (options (clearance outline) (anchor rect)) (primitives))
  (pad 3 smd rect (at -1.65 -1.5 90) (size 1.3 0.9) (layers B.Cu B.Paste B.Mask))
  (pad 1 smd rect (at -1.65 1.5 90) (size 1.3 0.9) (layers B.Cu B.Paste B.Mask)))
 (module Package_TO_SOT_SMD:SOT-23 (layer B.Cu) (at 155.5 116.5 90)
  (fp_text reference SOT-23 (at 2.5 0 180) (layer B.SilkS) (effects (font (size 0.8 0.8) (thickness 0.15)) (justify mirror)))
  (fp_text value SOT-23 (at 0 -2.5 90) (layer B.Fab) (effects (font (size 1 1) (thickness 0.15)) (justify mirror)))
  (pad 3 smd rect (at 1 0 90) (size 0.9 0.8) (layers B.Cu B.Paste B.Mask))
  (pad 2 smd rect (at -1 -0.95 90) (size 0.9 0.8) (layers B.Cu B.Paste B.Mask))
  (pad 1 smd rect (at -1 0.95 90) (size 0.9 0.8) (layers B.Cu B.Paste B.Mask)))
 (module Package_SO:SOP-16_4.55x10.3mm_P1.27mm (layer B.Cu) (at 171.5 114 90)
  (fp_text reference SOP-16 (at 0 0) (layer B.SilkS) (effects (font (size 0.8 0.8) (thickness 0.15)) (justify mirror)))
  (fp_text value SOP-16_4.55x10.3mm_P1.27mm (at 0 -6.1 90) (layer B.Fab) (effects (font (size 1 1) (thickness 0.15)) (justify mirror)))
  (pad 16 smd roundrect (at 3.25 4.445 90) (size 1.6 0.6) (layers B.Cu B.Paste B.Mask) (roundrect_rratio 0.25))
  (pad 15 smd roundrect (at 3.25 3.175 90) (size 1.6 0.6) (layers B.Cu B.Paste B.Mask) (roundrect_rratio 0.25))
  (pad 14 smd roundrect (at 3.25 1.905 90) (size 1.6 0.6) (layers B.Cu B.Paste B.Mask) (roundrect_rratio 0.25))
  (pad 13 smd roundrect (at 3.25 0.635 90) (size 1.6 0.6) (layers B.Cu B.Paste B.Mask) (roundrect_rratio 0.25))
  (pad 12 smd roundrect (at 3.25 -0.635 90) (size 1.6 0.6) (layers B.Cu B.Paste B.Mask) (roundrect_rratio 0.25))
  (pad 11 smd roundrect (at 3.25 -1.905 90) (size 1.6 0.6) (layers B.Cu B.Paste B.Mask) (roundrect_rratio 0.25))
  (pad 10 smd roundrect (at 3.25 -3.175 90) (size 1.6 0.6) (layers B.Cu B.Paste B.Mask) (roundrect_rratio 0.25))
  (pad 9 smd roundrect (at 3.25 -4.445 90) (size 1.6 0.6) (layers B.Cu B.Paste B.Mask) (roundrect_rratio 0.25))
  (pad 8 smd roundrect (at -3.25 -4.445 90) (size 1.6 0.6) (layers B.Cu B.Paste B.Mask) (roundrect_rratio 0.25))
  (pad 7 smd roundrect (at -3.25 -3.175 90) (size 1.6 0.6) (layers B.Cu B.Paste B.Mask) (roundrect_rratio 0.25))
  (pad 6 smd roundrect (at -3.25 -1.905 90) (size 1.6 0.6) (layers B.Cu B.Paste B.Mask) (roundrect_rratio 0.25))
  (pad 5 smd roundrect (at -3.25 -0.635 90) (size 1.6 0.6) (layers B.Cu B.Paste B.Mask) (roundrect_rratio 0.25))
  (pad 4 smd roundrect (at -3.25 0.635 90) (size 1.6 0.6) (layers B.Cu B.Paste B.Mask) (roundrect_rratio 0.25))
  (pad 3 smd roundrect (at -3.25 1.905 90) (size 1.6 0.6) (layers B.Cu B.Paste B.Mask) (roundrect_rratio 0.25))
  (pad 2 smd roundrect (at -3.25 3.175 90) (size 1.6 0.6) (layers B.Cu B.Paste B.Mask) (roundrect_rratio 0.25))
  (pad 1 smd roundrect (at -3.25 4.445 90) (size 1.6 0.6) (layers B.Cu B.Paste B.Mask) (roundrect_rratio 0.25)))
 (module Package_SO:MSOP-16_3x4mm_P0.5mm (layer B.Cu) (at 186.5 115 90)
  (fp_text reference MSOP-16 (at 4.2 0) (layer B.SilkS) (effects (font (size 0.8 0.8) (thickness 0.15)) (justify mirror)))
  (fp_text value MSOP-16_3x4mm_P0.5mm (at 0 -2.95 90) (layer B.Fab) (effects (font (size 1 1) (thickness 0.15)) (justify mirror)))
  (pad 16 smd roundrect (at 2.15 1.75 90) (size 1.45 0.3) (layers B.Cu B.Paste B.Mask) (roundrect_rratio 0.25))
  (pad 15 smd roundrect (at 2.15 1.25 90) (size 1.45 0.3) (layers B.Cu B.Paste B.Mask) (roundrect_rratio 0.25))
  (pad 14 smd roundrect (at 2.15 0.75 90) (size 1.45 0.3) (layers B.Cu B.Paste B.Mask) (roundrect_rratio 0.25))
  (pad 13 smd roundrect (at 2.15 0.25 90) (size 1.45 0.3) (layers B.Cu B.Paste B.Mask) (roundrect_rratio 0.25))
  (pad 12 smd roundrect (at 2.15 -0.25 90) (size 1.45 0.3) (layers B.Cu B.Paste B.Mask) (roundrect_rratio 0.25))
  (pad 11 smd roundrect (at 2.15 -0.75 90) (size 1.45 0.3) (layers B.Cu B.Paste B.Mask) (roundrect_rratio 0.25))
  (pad 10 smd roundrect (at 2.15 -1.25 90) (size 1.45 0.3) (layers B.Cu B.Paste B.Mask) (roundrect_rratio 0.25))
  (pad 9 smd roundrect (at 2.15 -1.75 90) (size 1.45 0.3) (layers B.Cu B.Paste B.Mask) (roundrect_rratio 0.25))
  (pad 8 smd roundrect (at -2.15 -1.75 90) (size 1.45 0.3) (layers B.Cu B.Paste B.Mask) (roundrect_rratio 0.25))
  (pad 7 smd roundrect (at -2.15 -1.25 90) (size 1.45 0.3) (layers B.Cu B.Paste B.Mask) (roundrect_rratio 0.25))
  (pad 6 smd roundrect (at -2.15 -0.75 90) (size 1.45 0.3) (layers B.Cu B.Paste B.Mask) (roundrect_rratio 0.25))
  (pad 5 smd roundrect (at -2.15 -0.25 90) (size 1.45 0.3) (layers B.Cu B.Paste B.Mask) (roundrect_rratio 0.25))
  (pad 4 smd roundrect (at -2.15 0.25 90) (size 1.45 0.3) (layers B.Cu B.Paste B.Mask) (roundrect_rratio 0.25))
  (pad 3 smd roundrect (at -2.15 0.75 90) (size 1.45 0.3) (layers B.Cu B.Paste B.Mask) (roundrect_rratio 0.25))
  (pad 2 smd roundrect (at -2.15 1.25 90) (size 1.45 0.3) (layers B.Cu B.Paste B.Mask) (roundrect_rratio 0.25))
  (pad 1 smd roundrect (at -2.15 1.75 90) (size 1.45 0.3) (layers B.Cu B.Paste B.Mask) (roundrect_rratio 0.25)))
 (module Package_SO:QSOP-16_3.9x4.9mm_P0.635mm (layer B.Cu) (at 180 114.5 90)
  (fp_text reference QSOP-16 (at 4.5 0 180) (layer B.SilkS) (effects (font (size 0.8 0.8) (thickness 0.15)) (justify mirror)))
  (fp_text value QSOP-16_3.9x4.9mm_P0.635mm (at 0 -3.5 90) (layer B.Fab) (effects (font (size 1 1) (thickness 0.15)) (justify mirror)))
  (pad 16 smd rect (at 2.6543 2.2225 90) (size 1.6 0.41) (layers B.Cu B.Paste B.Mask))
  (pad 15 smd rect (at 2.6543 1.5875 90) (size 1.6 0.41) (layers B.Cu B.Paste B.Mask))
  (pad 14 smd rect (at 2.6543 0.9525 90) (size 1.6 0.41) (layers B.Cu B.Paste B.Mask))
  (pad 13 smd rect (at 2.6543 0.3175 90) (size 1.6 0.41) (layers B.Cu B.Paste B.Mask))
  (pad 12 smd rect (at 2.6543 -0.3175 90) (size 1.6 0.41) (layers B.Cu B.Paste B.Mask))
  (pad 11 smd rect (at 2.6543 -0.9525 90) (size 1.6 0.41) (layers B.Cu B.Paste B.Mask))
  (pad 10 smd rect (at 2.6543 -1.5875 90) (size 1.6 0.41) (layers B.Cu B.Paste B.Mask))
  (pad 9 smd rect (at 2.6543 -2.2225 90) (size 1.6 0.41) (layers B.Cu B.Paste B.Mask))
  (pad 8 smd rect (at -2.6543 -2.2225 90) (size 1.6 0.41) (layers B.Cu B.Paste B.Mask))
  (pad 7 smd rect (at -2.6543 -1.5875 90) (size 1.6 0.41) (layers B.Cu B.Paste B.Mask))
  (pad 6 smd rect (at -2.6543 -0.9525 90) (size 1.6 0.41) (layers B.Cu B.Paste B.Mask))
  (pad 5 smd rect (at -2.6543 -0.3175 90) (size 1.6 0.41) (layers B.Cu B.Paste B.Mask))
  (pad 4 smd rect (at -2.6543 0.3175 90) (size 1.6 0.41) (layers B.Cu B.Paste B.Mask))
  (pad 3 smd rect (at -2.6543 0.9525 90) (size 1.6 0.41) (layers B.Cu B.Paste B.Mask))
  (pad 2 smd rect (at -2.6543 1.5875 90) (size 1.6 0.41) (layers B.Cu B.Paste B.Mask))
  (pad 1 smd rect (at -2.6543 2.2225 90) (size 1.6 0.41) (layers B.Cu B.Paste B.Mask)))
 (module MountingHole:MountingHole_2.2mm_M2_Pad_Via (layer F.Cu) (at 195 110)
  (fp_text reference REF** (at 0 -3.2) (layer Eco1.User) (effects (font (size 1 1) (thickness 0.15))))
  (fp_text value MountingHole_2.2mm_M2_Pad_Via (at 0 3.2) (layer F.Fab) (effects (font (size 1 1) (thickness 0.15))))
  (pad 1 thru_hole circle (at 1.166726 -1.166726) (size 0.7 0.7) (drill 0.4) (layers *.Cu *.Mask))
  (pad 1 thru_hole circle (at 0 -1.65) (size 0.7 0.7) (drill 0.4) (layers *.Cu *.Mask))
  (pad 1 thru_hole circle (at -1.166726 -1.166726) (size 0.7 0.7) (drill 0.4) (layers *.Cu *.Mask))
  (pad 1 thru_hole circle (at -1.65 0) (size 0.7 0.7) (drill 0.4) (layers *.Cu *.Mask))
  (pad 1 thru_hole circle (at -1.166726 1.166726) (size 0.7 0.7) (drill 0.4) (layers *.Cu *.Mask))
  (pad 1 thru_hole circle (at 0 1.65) (size 0.7 0.7) (drill 0.4) (layers *.Cu *.Mask))
  (pad 1 thru_hole circle (at 1.166726 1.166726) (size 0.7 0.7) (drill 0.4) (layers *.Cu *.Mask))
  (pad 1 thru_hole circle (at 1.65 0) (size 0.7 0.7) (drill 0.4) (layers *.Cu *.Mask))
  (pad 1 thru_hole circle (at 0 0) (size 4.4 4.4) (drill 2.2) (layers *.Cu *.Mask)))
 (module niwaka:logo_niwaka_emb (layer F.Cu) (at 170.5 113)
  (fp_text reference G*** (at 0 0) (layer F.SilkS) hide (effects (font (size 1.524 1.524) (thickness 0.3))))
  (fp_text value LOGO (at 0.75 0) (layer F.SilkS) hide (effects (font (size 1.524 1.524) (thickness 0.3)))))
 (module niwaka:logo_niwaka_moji (layer F.Cu) (at 187.5 117.5)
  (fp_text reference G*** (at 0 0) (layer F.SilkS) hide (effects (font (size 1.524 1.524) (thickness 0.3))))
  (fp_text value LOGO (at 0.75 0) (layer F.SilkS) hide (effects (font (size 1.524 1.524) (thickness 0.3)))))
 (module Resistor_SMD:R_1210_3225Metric (layer F.Cu) (at 160 117)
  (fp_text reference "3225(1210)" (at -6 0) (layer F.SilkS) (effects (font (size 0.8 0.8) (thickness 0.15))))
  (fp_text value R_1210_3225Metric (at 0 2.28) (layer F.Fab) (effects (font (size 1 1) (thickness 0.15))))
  (pad 2 smd roundrect (at 1.4 0) (size 1.25 2.65) (layers F.Cu F.Paste F.Mask) (roundrect_rratio 0.2))
  (pad 1 smd roundrect (at -1.4 0) (size 1.25 2.65) (layers F.Cu F.Paste F.Mask) (roundrect_rratio 0.2)))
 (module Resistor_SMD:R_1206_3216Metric (layer F.Cu) (at 160 113.75)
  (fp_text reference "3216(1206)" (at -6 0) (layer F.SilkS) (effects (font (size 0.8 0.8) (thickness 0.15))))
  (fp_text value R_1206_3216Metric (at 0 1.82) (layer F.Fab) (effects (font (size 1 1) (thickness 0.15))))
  (pad 2 smd roundrect (at 1.4 0) (size 1.25 1.75) (layers F.Cu F.Paste F.Mask) (roundrect_rratio 0.2))
  (pad 1 smd roundrect (at -1.4 0) (size 1.25 1.75) (layers F.Cu F.Paste F.Mask) (roundrect_rratio 0.2)))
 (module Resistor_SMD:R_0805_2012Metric (layer F.Cu) (at 160 111)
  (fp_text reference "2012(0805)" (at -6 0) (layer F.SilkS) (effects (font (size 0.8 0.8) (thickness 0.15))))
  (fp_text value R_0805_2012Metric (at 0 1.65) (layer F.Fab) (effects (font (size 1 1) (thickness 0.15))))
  (pad 1 smd roundrect (at -0.9375 0) (size 0.975 1.4) (layers F.Cu F.Paste F.Mask) (roundrect_rratio 0.25))
  (pad 2 smd roundrect (at 0.9375 0) (size 0.975 1.4) (layers F.Cu F.Paste F.Mask) (roundrect_rratio 0.25)))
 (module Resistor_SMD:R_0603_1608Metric (layer F.Cu) (at 148 117)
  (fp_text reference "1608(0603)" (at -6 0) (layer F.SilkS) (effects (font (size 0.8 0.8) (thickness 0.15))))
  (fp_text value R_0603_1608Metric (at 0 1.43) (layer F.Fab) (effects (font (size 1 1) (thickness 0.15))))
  (pad 1 smd roundrect (at -0.7875 0) (size 0.875 0.95) (layers F.Cu F.Paste F.Mask) (roundrect_rratio 0.25))
  (pad 2 smd roundrect (at 0.7875 0) (size 0.875 0.95) (layers F.Cu F.Paste F.Mask) (roundrect_rratio 0.25)))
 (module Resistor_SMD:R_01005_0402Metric (layer F.Cu) (at 148 111)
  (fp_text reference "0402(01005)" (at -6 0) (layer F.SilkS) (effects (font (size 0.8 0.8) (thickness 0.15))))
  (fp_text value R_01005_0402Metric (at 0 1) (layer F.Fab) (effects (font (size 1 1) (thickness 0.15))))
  (pad "" smd roundrect (at -0.275 0) (size 0.27 0.27) (layers F.Paste) (roundrect_rratio 0.25))
  (pad "" smd roundrect (at 0.275 0) (size 0.27 0.27) (layers F.Paste) (roundrect_rratio 0.25))
  (pad 1 smd roundrect (at -0.25 0) (size 0.4 0.3) (layers F.Cu F.Mask) (roundrect_rratio 0.25))
  (pad 2 smd roundrect (at 0.25 0) (size 0.4 0.3) (layers F.Cu F.Mask) (roundrect_rratio 0.25)))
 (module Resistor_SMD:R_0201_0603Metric (layer F.Cu) (at 148 113)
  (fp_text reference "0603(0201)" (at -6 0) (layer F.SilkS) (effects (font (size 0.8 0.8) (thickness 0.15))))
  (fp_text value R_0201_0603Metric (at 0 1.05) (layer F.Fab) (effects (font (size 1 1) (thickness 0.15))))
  (pad 2 smd roundrect (at 0.32 0) (size 0.46 0.4) (layers F.Cu F.Mask) (roundrect_rratio 0.25))
  (pad 1 smd roundrect (at -0.32 0) (size 0.46 0.4) (layers F.Cu F.Mask) (roundrect_rratio 0.25))
  (pad "" smd roundrect (at 0.345 0) (size 0.318 0.36) (layers F.Paste) (roundrect_rratio 0.25))
  (pad "" smd roundrect (at -0.345 0) (size 0.318 0.36) (layers F.Paste) (roundrect_rratio 0.25)))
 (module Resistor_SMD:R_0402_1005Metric (layer F.Cu) (at 148 115)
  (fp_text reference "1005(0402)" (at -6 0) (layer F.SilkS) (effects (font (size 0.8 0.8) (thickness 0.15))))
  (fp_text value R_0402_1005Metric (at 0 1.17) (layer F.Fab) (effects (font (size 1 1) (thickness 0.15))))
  (pad 1 smd roundrect (at -0.485 0) (size 0.59 0.64) (layers F.Cu F.Paste F.Mask) (roundrect_rratio 0.25))
  (pad 2 smd roundrect (at 0.485 0) (size 0.59 0.64) (layers F.Cu F.Paste F.Mask) (roundrect_rratio 0.25)))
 (gr_line (start 200 120) (end 100 120) (layer Edge.Cuts) (width 0.05))
 (gr_circle (center 103 119) (end 103.1 119) (layer Edge.Cuts) (width 0.05))
 (gr_circle (center 105 119) (end 105.15 119) (layer Edge.Cuts) (width 0.05))
 (gr_circle (center 107 119) (end 107.2 119) (layer Edge.Cuts) (width 0.05))
 (gr_circle (center 109 119) (end 109.25 119) (layer Edge.Cuts) (width 0.05))
 (gr_circle (center 119 119) (end 119.5 119) (layer Edge.Cuts) (width 0.05))
 (gr_circle (center 117 119) (end 117.45 119) (layer Edge.Cuts) (width 0.05))
 (gr_circle (center 114.9 119) (end 115.3 119) (layer Edge.Cuts) (width 0.05))
 (gr_circle (center 113 119) (end 113.35 119) (layer Edge.Cuts) (width 0.05))
 (gr_circle (center 111 119) (end 111.3 119) (layer Edge.Cuts) (width 0.05))
 (gr_line (start 100 120) (end 100 100) (layer Edge.Cuts) (width 0.05))
 (gr_line (start 200 100) (end 200 120) (layer Edge.Cuts) (width 0.05))
 (gr_line (start 100 100) (end 200 100) (layer Edge.Cuts) (width 0.05))
 (segment (start 103 111) (end 103 115) (width 0.1) (layer F.Cu) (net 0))
 (segment (start 105 111) (end 105 115) (width 0.15) (layer F.Cu) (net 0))
 (segment (start 107 111) (end 107 115) (width 0.2) (layer F.Cu) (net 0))
 (segment (start 109 111) (end 109 115) (width 0.25) (layer F.Cu) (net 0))
 (segment (start 111 111) (end 111 115) (width 0.3) (layer F.Cu) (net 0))
 (segment (start 113 111) (end 113 115) (width 0.35) (layer F.Cu) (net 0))
 (segment (start 117 111) (end 117 115) (width 0.45) (layer F.Cu) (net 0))
 (segment (start 119 111) (end 119 115) (width 0.5) (layer F.Cu) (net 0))
 (segment (start 115 111) (end 115 115) (width 0.4) (layer F.Cu) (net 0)))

